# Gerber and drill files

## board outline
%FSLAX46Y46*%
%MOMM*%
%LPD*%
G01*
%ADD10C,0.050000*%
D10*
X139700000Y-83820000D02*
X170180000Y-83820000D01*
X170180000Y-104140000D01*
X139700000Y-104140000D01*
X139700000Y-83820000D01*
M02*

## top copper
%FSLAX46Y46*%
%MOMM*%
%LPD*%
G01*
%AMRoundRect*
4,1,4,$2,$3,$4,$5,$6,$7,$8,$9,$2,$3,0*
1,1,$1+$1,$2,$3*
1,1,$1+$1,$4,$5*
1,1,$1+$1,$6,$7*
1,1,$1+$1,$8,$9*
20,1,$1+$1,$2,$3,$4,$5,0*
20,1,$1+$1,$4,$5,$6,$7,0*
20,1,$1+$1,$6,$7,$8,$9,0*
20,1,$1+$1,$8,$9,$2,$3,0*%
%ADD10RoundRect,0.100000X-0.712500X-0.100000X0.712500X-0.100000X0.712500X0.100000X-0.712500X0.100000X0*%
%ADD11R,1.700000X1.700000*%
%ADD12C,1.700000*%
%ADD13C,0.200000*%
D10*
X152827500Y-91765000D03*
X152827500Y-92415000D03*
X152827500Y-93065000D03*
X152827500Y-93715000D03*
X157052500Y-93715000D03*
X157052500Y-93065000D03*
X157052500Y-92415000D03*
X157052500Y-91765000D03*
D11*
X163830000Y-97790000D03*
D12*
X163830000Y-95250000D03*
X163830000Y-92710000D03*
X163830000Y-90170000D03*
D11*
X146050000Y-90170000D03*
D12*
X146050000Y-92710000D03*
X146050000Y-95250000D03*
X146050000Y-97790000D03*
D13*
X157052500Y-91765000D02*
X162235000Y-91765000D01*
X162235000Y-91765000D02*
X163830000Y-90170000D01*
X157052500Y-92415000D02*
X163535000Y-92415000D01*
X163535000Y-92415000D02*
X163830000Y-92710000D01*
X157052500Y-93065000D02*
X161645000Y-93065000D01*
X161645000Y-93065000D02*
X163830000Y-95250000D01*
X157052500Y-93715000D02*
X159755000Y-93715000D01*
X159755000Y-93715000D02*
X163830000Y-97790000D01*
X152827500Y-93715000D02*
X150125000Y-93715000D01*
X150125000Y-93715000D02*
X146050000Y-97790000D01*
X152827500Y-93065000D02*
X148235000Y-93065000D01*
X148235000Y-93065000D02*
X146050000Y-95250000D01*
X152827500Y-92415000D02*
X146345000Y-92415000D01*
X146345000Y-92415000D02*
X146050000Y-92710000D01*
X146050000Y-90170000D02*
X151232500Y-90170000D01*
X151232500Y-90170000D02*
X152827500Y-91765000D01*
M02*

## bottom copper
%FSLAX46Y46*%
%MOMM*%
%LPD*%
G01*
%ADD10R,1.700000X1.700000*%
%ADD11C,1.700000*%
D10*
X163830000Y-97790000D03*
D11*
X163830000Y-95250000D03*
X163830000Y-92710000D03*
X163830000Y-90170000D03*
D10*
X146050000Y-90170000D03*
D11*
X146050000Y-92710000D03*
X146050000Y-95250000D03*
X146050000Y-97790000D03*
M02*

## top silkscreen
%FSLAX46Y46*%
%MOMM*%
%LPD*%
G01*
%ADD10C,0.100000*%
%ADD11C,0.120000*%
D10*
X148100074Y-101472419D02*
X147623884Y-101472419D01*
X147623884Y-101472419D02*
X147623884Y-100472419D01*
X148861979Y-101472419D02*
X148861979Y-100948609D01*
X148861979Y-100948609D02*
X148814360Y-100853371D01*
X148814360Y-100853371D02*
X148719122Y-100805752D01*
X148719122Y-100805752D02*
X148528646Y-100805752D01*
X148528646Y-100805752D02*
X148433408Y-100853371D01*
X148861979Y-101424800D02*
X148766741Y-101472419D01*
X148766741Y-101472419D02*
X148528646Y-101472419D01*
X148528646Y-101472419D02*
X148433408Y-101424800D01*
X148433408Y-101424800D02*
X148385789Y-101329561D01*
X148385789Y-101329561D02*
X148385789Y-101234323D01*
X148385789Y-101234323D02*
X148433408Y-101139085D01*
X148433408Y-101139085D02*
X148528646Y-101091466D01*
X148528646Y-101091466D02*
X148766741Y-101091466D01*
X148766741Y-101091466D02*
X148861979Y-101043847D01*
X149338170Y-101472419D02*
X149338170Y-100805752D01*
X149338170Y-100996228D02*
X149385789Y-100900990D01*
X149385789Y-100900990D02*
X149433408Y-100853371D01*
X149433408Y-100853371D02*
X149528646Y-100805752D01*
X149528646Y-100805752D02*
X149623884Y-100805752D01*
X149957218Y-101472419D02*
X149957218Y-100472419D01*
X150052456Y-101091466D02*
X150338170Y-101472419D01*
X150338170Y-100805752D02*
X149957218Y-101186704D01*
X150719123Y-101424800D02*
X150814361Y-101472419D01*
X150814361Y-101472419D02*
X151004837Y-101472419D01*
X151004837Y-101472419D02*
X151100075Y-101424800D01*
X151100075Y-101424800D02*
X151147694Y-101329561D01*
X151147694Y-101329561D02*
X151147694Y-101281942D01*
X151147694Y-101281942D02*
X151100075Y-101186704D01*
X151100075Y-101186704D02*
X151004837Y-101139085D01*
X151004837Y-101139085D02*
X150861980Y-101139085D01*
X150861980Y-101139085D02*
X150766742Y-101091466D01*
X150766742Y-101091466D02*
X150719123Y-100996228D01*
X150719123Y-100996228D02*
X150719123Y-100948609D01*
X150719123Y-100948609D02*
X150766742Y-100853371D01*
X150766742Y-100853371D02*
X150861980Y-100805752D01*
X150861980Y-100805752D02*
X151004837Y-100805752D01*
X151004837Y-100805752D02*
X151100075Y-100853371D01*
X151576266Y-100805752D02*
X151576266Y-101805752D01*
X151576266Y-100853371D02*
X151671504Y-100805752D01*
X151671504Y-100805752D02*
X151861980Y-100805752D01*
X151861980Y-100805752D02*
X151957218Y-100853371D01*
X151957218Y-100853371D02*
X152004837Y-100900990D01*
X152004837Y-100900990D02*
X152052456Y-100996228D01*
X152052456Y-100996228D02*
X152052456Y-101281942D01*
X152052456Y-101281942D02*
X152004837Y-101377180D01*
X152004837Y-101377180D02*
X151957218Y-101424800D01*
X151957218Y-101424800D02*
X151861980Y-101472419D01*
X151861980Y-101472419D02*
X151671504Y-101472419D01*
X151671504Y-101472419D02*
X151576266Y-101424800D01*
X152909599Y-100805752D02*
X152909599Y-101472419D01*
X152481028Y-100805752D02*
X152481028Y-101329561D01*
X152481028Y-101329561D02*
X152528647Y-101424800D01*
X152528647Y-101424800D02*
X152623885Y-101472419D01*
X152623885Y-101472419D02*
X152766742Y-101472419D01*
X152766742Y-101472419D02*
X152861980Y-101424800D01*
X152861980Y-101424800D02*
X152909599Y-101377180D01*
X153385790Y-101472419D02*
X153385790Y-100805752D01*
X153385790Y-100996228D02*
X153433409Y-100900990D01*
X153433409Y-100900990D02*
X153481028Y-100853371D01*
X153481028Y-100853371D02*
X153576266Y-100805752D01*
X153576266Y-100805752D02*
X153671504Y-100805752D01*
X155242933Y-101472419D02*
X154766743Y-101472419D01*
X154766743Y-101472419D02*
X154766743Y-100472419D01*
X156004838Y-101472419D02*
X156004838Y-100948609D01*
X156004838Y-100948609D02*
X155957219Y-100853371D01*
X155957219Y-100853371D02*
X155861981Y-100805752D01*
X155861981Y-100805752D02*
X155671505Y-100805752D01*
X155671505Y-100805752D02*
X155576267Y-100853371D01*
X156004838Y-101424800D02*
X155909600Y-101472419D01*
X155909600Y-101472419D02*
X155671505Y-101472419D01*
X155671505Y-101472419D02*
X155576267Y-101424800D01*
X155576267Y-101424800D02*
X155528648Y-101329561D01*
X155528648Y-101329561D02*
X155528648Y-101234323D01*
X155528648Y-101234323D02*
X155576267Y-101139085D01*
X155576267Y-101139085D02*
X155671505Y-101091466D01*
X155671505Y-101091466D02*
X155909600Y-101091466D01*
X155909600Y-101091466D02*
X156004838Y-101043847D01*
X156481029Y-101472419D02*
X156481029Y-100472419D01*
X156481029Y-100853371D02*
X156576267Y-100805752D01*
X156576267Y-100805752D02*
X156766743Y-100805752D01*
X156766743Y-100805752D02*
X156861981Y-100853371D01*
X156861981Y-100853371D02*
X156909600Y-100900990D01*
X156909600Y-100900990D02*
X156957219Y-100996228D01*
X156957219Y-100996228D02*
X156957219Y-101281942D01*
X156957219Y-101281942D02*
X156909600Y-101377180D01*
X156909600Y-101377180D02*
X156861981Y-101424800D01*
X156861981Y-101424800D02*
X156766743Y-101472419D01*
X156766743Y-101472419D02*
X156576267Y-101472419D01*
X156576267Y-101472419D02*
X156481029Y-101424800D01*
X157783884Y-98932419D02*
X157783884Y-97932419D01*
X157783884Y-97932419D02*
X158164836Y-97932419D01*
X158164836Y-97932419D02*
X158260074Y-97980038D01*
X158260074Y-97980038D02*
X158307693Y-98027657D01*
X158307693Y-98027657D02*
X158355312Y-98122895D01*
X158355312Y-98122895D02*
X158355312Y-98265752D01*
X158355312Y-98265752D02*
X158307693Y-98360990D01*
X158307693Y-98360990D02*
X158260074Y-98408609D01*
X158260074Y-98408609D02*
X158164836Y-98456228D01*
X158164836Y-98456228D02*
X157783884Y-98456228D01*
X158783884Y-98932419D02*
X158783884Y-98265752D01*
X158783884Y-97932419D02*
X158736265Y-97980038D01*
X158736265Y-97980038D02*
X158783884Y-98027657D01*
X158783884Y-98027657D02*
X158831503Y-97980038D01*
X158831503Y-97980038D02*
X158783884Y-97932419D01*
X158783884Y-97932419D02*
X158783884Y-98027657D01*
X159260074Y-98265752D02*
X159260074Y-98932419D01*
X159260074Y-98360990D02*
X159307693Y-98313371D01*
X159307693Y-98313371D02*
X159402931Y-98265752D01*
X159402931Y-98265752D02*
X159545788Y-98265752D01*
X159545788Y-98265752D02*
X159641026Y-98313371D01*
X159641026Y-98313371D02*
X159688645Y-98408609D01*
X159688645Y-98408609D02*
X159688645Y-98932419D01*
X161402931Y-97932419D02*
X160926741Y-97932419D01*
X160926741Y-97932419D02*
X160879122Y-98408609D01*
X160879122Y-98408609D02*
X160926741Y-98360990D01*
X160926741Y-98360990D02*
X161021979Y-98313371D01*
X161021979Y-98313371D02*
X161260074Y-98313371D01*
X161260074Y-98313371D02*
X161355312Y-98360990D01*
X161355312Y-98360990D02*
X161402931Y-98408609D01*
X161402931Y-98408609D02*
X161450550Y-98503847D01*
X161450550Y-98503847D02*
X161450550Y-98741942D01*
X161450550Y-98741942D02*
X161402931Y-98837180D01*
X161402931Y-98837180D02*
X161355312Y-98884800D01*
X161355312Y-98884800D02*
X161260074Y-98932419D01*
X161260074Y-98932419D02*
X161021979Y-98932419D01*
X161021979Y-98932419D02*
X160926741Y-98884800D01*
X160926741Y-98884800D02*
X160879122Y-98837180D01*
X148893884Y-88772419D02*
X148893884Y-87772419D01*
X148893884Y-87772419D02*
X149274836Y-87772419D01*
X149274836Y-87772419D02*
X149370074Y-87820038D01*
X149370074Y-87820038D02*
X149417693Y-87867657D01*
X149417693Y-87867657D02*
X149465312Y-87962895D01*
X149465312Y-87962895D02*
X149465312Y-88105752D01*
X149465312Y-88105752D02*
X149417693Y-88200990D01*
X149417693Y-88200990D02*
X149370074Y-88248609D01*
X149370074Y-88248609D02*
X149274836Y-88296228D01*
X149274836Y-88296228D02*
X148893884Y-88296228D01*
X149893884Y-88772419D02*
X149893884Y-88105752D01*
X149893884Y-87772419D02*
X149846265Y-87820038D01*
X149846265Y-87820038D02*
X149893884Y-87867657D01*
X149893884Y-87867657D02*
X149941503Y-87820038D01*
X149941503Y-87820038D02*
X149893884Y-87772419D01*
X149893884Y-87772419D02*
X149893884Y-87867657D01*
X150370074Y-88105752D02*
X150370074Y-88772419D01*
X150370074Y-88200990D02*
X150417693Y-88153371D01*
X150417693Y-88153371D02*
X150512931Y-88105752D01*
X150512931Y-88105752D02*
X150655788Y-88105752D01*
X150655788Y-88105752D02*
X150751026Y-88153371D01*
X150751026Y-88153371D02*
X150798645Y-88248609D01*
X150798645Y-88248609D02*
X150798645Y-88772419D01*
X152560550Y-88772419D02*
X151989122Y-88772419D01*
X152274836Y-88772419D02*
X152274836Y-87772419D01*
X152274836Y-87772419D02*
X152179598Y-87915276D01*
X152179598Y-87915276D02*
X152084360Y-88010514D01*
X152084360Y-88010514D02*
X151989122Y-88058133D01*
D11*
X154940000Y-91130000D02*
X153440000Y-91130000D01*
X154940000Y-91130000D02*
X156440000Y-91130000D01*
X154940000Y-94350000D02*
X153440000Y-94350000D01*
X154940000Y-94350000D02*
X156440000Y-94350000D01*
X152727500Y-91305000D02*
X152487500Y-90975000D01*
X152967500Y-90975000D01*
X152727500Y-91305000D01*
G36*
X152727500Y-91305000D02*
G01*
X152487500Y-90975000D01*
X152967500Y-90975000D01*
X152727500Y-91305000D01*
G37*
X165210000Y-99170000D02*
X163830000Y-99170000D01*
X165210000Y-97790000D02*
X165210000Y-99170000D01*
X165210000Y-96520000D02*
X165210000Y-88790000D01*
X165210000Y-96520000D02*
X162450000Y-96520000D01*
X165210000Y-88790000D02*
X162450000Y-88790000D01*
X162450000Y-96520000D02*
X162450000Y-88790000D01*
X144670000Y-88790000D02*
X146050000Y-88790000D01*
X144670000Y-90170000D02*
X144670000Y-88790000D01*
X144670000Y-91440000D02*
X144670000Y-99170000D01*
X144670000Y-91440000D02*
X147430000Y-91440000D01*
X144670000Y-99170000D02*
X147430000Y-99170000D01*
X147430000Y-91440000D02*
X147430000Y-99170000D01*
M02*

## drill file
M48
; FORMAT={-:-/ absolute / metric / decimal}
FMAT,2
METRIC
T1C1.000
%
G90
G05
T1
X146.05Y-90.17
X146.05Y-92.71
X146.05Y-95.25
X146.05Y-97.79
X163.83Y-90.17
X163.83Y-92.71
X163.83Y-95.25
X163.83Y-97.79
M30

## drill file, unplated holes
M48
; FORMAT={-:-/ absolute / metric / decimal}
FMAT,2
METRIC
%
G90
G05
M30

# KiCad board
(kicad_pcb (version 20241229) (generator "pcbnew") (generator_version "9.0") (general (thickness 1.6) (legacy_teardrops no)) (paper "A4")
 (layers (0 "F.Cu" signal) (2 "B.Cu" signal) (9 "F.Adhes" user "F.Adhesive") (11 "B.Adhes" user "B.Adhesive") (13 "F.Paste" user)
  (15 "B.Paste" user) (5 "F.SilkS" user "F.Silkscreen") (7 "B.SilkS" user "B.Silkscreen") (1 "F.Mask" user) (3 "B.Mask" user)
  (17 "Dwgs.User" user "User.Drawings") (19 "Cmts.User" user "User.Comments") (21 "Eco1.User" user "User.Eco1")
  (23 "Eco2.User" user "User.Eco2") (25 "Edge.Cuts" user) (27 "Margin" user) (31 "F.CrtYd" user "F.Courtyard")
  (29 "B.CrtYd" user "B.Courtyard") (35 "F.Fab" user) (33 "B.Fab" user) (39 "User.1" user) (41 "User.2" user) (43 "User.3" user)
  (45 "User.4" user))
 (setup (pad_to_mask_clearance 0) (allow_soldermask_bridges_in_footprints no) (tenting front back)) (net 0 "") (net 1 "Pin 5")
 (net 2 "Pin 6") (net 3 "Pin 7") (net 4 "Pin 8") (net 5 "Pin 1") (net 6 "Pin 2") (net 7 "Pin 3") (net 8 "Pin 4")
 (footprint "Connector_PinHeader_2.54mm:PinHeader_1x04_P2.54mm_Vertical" (layer "F.Cu") (at 163.83 97.79 180)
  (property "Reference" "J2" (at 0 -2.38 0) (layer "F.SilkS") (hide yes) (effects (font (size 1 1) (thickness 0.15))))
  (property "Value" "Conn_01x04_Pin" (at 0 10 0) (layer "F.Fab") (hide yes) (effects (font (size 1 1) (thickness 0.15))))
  (fp_line (start 1.38 1.27) (end 1.38 9) (stroke (width 0.12) (type solid)) (layer "F.SilkS"))
  (fp_line (start -1.38 9) (end 1.38 9) (stroke (width 0.12) (type solid)) (layer "F.SilkS"))
  (fp_line (start -1.38 1.27) (end 1.38 1.27) (stroke (width 0.12) (type solid)) (layer "F.SilkS"))
  (fp_line (start -1.38 1.27) (end -1.38 9) (stroke (width 0.12) (type solid)) (layer "F.SilkS"))
  (fp_line (start -1.38 0) (end -1.38 -1.38) (stroke (width 0.12) (type solid)) (layer "F.SilkS"))
  (fp_line (start -1.38 -1.38) (end 0 -1.38) (stroke (width 0.12) (type solid)) (layer "F.SilkS"))
  (pad "1" thru_hole rect (at 0 0 180) (size 1.7 1.7) (drill 1) (layers "*.Cu" "*.Mask") (remove_unused_layers no) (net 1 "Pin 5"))
  (pad "2" thru_hole circle (at 0 2.54 180) (size 1.7 1.7) (drill 1) (layers "*.Cu" "*.Mask") (remove_unused_layers no) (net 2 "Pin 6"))
  (pad "3" thru_hole circle (at 0 5.08 180) (size 1.7 1.7) (drill 1) (layers "*.Cu" "*.Mask") (remove_unused_layers no) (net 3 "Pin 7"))
  (pad "4" thru_hole circle (at 0 7.62 180) (size 1.7 1.7) (drill 1) (layers "*.Cu" "*.Mask") (remove_unused_layers no) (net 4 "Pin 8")))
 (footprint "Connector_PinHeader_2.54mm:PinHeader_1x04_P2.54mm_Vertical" (layer "F.Cu") (at 146.05 90.17)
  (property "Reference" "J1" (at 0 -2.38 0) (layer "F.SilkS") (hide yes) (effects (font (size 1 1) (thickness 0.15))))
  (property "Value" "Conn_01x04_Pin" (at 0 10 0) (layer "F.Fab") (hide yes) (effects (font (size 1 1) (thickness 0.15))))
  (fp_line (start -1.38 -1.38) (end 0 -1.38) (stroke (width 0.12) (type solid)) (layer "F.SilkS"))
  (fp_line (start -1.38 0) (end -1.38 -1.38) (stroke (width 0.12) (type solid)) (layer "F.SilkS"))
  (fp_line (start -1.38 1.27) (end -1.38 9) (stroke (width 0.12) (type solid)) (layer "F.SilkS"))
  (fp_line (start -1.38 1.27) (end 1.38 1.27) (stroke (width 0.12) (type solid)) (layer "F.SilkS"))
  (fp_line (start -1.38 9) (end 1.38 9) (stroke (width 0.12) (type solid)) (layer "F.SilkS"))
  (fp_line (start 1.38 1.27) (end 1.38 9) (stroke (width 0.12) (type solid)) (layer "F.SilkS"))
  (pad "1" thru_hole rect (at 0 0) (size 1.7 1.7) (drill 1) (layers "*.Cu" "*.Mask") (remove_unused_layers no) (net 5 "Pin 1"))
  (pad "2" thru_hole circle (at 0 2.54) (size 1.7 1.7) (drill 1) (layers "*.Cu" "*.Mask") (remove_unused_layers no) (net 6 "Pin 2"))
  (pad "3" thru_hole circle (at 0 5.08) (size 1.7 1.7) (drill 1) (layers "*.Cu" "*.Mask") (remove_unused_layers no) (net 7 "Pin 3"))
  (pad "4" thru_hole circle (at 0 7.62) (size 1.7 1.7) (drill 1) (layers "*.Cu" "*.Mask") (remove_unused_layers no) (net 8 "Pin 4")))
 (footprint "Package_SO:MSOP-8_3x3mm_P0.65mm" (layer "F.Cu") (at 154.94 92.74)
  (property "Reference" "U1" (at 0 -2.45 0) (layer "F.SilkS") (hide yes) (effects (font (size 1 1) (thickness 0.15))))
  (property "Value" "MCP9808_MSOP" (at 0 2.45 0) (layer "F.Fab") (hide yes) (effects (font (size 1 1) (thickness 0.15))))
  (fp_line (start 0 -1.61) (end -1.5 -1.61) (stroke (width 0.12) (type solid)) (layer "F.SilkS"))
  (fp_line (start 0 -1.61) (end 1.5 -1.61) (stroke (width 0.12) (type solid)) (layer "F.SilkS"))
  (fp_line (start 0 1.61) (end -1.5 1.61) (stroke (width 0.12) (type solid)) (layer "F.SilkS"))
  (fp_line (start 0 1.61) (end 1.5 1.61) (stroke (width 0.12) (type solid)) (layer "F.SilkS"))
  (fp_poly
   (pts (xy -2.2125 -1.435) (xy -2.4525 -1.765) (xy -1.9725 -1.765)) (stroke (width 0.12) (type solid)) (fill yes) (layer "F.SilkS"))
  (pad "1" smd roundrect (at -2.1125 -0.975) (size 1.625 0.4) (layers "F.Cu" "F.Mask" "F.Paste") (roundrect_rratio 0.25) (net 5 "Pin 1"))
  (pad "2" smd roundrect (at -2.1125 -0.325) (size 1.625 0.4) (layers "F.Cu" "F.Mask" "F.Paste") (roundrect_rratio 0.25) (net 6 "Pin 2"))
  (pad "3" smd roundrect (at -2.1125 0.325) (size 1.625 0.4) (layers "F.Cu" "F.Mask" "F.Paste") (roundrect_rratio 0.25) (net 7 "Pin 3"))
  (pad "4" smd roundrect (at -2.1125 0.975) (size 1.625 0.4) (layers "F.Cu" "F.Mask" "F.Paste") (roundrect_rratio 0.25) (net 8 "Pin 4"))
  (pad "5" smd roundrect (at 2.1125 0.975) (size 1.625 0.4) (layers "F.Cu" "F.Mask" "F.Paste") (roundrect_rratio 0.25) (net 1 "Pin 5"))
  (pad "6" smd roundrect (at 2.1125 0.325) (size 1.625 0.4) (layers "F.Cu" "F.Mask" "F.Paste") (roundrect_rratio 0.25) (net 2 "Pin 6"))
  (pad "7" smd roundrect (at 2.1125 -0.325) (size 1.625 0.4) (layers "F.Cu" "F.Mask" "F.Paste") (roundrect_rratio 0.25) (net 3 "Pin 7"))
  (pad "8" smd roundrect (at 2.1125 -0.975) (size 1.625 0.4) (layers "F.Cu" "F.Mask" "F.Paste") (roundrect_rratio 0.25) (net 4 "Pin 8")))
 (gr_rect (start 139.7 83.82) (end 170.18 104.14) (stroke (width 0.05) (type default)) (fill no) (layer "Edge.Cuts"))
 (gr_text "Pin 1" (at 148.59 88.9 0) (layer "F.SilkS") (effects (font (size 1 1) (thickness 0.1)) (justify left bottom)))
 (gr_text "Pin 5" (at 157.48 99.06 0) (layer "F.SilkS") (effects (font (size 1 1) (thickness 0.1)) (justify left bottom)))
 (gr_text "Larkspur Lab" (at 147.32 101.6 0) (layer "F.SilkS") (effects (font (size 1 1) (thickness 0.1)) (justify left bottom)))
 (segment (start 146.345 92.415) (end 146.05 92.71) (width 0.2) (layer "F.Cu") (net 6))
 (segment (start 152.8275 92.415) (end 146.345 92.415) (width 0.2) (layer "F.Cu") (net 6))
 (segment (start 151.2325 90.17) (end 152.8275 91.765) (width 0.2) (layer "F.Cu") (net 5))
 (segment (start 146.05 90.17) (end 151.2325 90.17) (width 0.2) (layer "F.Cu") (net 5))
 (segment (start 148.235 93.065) (end 146.05 95.25) (width 0.2) (layer "F.Cu") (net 7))
 (segment (start 152.8275 93.065) (end 148.235 93.065) (width 0.2) (layer "F.Cu") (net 7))
 (segment (start 152.8275 93.715) (end 150.125 93.715) (width 0.2) (layer "F.Cu") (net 8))
 (segment (start 150.125 93.715) (end 146.05 97.79) (width 0.2) (layer "F.Cu") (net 8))
 (segment (start 159.755 93.715) (end 163.83 97.79) (width 0.2) (layer "F.Cu") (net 1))
 (segment (start 157.0525 93.715) (end 159.755 93.715) (width 0.2) (layer "F.Cu") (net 1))
 (segment (start 162.235 91.765) (end 163.83 90.17) (width 0.2) (layer "F.Cu") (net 4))
 (segment (start 157.0525 91.765) (end 162.235 91.765) (width 0.2) (layer "F.Cu") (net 4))
 (segment (start 161.645 93.065) (end 163.83 95.25) (width 0.2) (layer "F.Cu") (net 2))
 (segment (start 157.0525 93.065) (end 161.645 93.065) (width 0.2) (layer "F.Cu") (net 2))
 (segment (start 157.0525 92.415) (end 163.535 92.415) (width 0.2) (layer "F.Cu") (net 3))
 (segment (start 163.535 92.415) (end 163.83 92.71) (width 0.2) (layer "F.Cu") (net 3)))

